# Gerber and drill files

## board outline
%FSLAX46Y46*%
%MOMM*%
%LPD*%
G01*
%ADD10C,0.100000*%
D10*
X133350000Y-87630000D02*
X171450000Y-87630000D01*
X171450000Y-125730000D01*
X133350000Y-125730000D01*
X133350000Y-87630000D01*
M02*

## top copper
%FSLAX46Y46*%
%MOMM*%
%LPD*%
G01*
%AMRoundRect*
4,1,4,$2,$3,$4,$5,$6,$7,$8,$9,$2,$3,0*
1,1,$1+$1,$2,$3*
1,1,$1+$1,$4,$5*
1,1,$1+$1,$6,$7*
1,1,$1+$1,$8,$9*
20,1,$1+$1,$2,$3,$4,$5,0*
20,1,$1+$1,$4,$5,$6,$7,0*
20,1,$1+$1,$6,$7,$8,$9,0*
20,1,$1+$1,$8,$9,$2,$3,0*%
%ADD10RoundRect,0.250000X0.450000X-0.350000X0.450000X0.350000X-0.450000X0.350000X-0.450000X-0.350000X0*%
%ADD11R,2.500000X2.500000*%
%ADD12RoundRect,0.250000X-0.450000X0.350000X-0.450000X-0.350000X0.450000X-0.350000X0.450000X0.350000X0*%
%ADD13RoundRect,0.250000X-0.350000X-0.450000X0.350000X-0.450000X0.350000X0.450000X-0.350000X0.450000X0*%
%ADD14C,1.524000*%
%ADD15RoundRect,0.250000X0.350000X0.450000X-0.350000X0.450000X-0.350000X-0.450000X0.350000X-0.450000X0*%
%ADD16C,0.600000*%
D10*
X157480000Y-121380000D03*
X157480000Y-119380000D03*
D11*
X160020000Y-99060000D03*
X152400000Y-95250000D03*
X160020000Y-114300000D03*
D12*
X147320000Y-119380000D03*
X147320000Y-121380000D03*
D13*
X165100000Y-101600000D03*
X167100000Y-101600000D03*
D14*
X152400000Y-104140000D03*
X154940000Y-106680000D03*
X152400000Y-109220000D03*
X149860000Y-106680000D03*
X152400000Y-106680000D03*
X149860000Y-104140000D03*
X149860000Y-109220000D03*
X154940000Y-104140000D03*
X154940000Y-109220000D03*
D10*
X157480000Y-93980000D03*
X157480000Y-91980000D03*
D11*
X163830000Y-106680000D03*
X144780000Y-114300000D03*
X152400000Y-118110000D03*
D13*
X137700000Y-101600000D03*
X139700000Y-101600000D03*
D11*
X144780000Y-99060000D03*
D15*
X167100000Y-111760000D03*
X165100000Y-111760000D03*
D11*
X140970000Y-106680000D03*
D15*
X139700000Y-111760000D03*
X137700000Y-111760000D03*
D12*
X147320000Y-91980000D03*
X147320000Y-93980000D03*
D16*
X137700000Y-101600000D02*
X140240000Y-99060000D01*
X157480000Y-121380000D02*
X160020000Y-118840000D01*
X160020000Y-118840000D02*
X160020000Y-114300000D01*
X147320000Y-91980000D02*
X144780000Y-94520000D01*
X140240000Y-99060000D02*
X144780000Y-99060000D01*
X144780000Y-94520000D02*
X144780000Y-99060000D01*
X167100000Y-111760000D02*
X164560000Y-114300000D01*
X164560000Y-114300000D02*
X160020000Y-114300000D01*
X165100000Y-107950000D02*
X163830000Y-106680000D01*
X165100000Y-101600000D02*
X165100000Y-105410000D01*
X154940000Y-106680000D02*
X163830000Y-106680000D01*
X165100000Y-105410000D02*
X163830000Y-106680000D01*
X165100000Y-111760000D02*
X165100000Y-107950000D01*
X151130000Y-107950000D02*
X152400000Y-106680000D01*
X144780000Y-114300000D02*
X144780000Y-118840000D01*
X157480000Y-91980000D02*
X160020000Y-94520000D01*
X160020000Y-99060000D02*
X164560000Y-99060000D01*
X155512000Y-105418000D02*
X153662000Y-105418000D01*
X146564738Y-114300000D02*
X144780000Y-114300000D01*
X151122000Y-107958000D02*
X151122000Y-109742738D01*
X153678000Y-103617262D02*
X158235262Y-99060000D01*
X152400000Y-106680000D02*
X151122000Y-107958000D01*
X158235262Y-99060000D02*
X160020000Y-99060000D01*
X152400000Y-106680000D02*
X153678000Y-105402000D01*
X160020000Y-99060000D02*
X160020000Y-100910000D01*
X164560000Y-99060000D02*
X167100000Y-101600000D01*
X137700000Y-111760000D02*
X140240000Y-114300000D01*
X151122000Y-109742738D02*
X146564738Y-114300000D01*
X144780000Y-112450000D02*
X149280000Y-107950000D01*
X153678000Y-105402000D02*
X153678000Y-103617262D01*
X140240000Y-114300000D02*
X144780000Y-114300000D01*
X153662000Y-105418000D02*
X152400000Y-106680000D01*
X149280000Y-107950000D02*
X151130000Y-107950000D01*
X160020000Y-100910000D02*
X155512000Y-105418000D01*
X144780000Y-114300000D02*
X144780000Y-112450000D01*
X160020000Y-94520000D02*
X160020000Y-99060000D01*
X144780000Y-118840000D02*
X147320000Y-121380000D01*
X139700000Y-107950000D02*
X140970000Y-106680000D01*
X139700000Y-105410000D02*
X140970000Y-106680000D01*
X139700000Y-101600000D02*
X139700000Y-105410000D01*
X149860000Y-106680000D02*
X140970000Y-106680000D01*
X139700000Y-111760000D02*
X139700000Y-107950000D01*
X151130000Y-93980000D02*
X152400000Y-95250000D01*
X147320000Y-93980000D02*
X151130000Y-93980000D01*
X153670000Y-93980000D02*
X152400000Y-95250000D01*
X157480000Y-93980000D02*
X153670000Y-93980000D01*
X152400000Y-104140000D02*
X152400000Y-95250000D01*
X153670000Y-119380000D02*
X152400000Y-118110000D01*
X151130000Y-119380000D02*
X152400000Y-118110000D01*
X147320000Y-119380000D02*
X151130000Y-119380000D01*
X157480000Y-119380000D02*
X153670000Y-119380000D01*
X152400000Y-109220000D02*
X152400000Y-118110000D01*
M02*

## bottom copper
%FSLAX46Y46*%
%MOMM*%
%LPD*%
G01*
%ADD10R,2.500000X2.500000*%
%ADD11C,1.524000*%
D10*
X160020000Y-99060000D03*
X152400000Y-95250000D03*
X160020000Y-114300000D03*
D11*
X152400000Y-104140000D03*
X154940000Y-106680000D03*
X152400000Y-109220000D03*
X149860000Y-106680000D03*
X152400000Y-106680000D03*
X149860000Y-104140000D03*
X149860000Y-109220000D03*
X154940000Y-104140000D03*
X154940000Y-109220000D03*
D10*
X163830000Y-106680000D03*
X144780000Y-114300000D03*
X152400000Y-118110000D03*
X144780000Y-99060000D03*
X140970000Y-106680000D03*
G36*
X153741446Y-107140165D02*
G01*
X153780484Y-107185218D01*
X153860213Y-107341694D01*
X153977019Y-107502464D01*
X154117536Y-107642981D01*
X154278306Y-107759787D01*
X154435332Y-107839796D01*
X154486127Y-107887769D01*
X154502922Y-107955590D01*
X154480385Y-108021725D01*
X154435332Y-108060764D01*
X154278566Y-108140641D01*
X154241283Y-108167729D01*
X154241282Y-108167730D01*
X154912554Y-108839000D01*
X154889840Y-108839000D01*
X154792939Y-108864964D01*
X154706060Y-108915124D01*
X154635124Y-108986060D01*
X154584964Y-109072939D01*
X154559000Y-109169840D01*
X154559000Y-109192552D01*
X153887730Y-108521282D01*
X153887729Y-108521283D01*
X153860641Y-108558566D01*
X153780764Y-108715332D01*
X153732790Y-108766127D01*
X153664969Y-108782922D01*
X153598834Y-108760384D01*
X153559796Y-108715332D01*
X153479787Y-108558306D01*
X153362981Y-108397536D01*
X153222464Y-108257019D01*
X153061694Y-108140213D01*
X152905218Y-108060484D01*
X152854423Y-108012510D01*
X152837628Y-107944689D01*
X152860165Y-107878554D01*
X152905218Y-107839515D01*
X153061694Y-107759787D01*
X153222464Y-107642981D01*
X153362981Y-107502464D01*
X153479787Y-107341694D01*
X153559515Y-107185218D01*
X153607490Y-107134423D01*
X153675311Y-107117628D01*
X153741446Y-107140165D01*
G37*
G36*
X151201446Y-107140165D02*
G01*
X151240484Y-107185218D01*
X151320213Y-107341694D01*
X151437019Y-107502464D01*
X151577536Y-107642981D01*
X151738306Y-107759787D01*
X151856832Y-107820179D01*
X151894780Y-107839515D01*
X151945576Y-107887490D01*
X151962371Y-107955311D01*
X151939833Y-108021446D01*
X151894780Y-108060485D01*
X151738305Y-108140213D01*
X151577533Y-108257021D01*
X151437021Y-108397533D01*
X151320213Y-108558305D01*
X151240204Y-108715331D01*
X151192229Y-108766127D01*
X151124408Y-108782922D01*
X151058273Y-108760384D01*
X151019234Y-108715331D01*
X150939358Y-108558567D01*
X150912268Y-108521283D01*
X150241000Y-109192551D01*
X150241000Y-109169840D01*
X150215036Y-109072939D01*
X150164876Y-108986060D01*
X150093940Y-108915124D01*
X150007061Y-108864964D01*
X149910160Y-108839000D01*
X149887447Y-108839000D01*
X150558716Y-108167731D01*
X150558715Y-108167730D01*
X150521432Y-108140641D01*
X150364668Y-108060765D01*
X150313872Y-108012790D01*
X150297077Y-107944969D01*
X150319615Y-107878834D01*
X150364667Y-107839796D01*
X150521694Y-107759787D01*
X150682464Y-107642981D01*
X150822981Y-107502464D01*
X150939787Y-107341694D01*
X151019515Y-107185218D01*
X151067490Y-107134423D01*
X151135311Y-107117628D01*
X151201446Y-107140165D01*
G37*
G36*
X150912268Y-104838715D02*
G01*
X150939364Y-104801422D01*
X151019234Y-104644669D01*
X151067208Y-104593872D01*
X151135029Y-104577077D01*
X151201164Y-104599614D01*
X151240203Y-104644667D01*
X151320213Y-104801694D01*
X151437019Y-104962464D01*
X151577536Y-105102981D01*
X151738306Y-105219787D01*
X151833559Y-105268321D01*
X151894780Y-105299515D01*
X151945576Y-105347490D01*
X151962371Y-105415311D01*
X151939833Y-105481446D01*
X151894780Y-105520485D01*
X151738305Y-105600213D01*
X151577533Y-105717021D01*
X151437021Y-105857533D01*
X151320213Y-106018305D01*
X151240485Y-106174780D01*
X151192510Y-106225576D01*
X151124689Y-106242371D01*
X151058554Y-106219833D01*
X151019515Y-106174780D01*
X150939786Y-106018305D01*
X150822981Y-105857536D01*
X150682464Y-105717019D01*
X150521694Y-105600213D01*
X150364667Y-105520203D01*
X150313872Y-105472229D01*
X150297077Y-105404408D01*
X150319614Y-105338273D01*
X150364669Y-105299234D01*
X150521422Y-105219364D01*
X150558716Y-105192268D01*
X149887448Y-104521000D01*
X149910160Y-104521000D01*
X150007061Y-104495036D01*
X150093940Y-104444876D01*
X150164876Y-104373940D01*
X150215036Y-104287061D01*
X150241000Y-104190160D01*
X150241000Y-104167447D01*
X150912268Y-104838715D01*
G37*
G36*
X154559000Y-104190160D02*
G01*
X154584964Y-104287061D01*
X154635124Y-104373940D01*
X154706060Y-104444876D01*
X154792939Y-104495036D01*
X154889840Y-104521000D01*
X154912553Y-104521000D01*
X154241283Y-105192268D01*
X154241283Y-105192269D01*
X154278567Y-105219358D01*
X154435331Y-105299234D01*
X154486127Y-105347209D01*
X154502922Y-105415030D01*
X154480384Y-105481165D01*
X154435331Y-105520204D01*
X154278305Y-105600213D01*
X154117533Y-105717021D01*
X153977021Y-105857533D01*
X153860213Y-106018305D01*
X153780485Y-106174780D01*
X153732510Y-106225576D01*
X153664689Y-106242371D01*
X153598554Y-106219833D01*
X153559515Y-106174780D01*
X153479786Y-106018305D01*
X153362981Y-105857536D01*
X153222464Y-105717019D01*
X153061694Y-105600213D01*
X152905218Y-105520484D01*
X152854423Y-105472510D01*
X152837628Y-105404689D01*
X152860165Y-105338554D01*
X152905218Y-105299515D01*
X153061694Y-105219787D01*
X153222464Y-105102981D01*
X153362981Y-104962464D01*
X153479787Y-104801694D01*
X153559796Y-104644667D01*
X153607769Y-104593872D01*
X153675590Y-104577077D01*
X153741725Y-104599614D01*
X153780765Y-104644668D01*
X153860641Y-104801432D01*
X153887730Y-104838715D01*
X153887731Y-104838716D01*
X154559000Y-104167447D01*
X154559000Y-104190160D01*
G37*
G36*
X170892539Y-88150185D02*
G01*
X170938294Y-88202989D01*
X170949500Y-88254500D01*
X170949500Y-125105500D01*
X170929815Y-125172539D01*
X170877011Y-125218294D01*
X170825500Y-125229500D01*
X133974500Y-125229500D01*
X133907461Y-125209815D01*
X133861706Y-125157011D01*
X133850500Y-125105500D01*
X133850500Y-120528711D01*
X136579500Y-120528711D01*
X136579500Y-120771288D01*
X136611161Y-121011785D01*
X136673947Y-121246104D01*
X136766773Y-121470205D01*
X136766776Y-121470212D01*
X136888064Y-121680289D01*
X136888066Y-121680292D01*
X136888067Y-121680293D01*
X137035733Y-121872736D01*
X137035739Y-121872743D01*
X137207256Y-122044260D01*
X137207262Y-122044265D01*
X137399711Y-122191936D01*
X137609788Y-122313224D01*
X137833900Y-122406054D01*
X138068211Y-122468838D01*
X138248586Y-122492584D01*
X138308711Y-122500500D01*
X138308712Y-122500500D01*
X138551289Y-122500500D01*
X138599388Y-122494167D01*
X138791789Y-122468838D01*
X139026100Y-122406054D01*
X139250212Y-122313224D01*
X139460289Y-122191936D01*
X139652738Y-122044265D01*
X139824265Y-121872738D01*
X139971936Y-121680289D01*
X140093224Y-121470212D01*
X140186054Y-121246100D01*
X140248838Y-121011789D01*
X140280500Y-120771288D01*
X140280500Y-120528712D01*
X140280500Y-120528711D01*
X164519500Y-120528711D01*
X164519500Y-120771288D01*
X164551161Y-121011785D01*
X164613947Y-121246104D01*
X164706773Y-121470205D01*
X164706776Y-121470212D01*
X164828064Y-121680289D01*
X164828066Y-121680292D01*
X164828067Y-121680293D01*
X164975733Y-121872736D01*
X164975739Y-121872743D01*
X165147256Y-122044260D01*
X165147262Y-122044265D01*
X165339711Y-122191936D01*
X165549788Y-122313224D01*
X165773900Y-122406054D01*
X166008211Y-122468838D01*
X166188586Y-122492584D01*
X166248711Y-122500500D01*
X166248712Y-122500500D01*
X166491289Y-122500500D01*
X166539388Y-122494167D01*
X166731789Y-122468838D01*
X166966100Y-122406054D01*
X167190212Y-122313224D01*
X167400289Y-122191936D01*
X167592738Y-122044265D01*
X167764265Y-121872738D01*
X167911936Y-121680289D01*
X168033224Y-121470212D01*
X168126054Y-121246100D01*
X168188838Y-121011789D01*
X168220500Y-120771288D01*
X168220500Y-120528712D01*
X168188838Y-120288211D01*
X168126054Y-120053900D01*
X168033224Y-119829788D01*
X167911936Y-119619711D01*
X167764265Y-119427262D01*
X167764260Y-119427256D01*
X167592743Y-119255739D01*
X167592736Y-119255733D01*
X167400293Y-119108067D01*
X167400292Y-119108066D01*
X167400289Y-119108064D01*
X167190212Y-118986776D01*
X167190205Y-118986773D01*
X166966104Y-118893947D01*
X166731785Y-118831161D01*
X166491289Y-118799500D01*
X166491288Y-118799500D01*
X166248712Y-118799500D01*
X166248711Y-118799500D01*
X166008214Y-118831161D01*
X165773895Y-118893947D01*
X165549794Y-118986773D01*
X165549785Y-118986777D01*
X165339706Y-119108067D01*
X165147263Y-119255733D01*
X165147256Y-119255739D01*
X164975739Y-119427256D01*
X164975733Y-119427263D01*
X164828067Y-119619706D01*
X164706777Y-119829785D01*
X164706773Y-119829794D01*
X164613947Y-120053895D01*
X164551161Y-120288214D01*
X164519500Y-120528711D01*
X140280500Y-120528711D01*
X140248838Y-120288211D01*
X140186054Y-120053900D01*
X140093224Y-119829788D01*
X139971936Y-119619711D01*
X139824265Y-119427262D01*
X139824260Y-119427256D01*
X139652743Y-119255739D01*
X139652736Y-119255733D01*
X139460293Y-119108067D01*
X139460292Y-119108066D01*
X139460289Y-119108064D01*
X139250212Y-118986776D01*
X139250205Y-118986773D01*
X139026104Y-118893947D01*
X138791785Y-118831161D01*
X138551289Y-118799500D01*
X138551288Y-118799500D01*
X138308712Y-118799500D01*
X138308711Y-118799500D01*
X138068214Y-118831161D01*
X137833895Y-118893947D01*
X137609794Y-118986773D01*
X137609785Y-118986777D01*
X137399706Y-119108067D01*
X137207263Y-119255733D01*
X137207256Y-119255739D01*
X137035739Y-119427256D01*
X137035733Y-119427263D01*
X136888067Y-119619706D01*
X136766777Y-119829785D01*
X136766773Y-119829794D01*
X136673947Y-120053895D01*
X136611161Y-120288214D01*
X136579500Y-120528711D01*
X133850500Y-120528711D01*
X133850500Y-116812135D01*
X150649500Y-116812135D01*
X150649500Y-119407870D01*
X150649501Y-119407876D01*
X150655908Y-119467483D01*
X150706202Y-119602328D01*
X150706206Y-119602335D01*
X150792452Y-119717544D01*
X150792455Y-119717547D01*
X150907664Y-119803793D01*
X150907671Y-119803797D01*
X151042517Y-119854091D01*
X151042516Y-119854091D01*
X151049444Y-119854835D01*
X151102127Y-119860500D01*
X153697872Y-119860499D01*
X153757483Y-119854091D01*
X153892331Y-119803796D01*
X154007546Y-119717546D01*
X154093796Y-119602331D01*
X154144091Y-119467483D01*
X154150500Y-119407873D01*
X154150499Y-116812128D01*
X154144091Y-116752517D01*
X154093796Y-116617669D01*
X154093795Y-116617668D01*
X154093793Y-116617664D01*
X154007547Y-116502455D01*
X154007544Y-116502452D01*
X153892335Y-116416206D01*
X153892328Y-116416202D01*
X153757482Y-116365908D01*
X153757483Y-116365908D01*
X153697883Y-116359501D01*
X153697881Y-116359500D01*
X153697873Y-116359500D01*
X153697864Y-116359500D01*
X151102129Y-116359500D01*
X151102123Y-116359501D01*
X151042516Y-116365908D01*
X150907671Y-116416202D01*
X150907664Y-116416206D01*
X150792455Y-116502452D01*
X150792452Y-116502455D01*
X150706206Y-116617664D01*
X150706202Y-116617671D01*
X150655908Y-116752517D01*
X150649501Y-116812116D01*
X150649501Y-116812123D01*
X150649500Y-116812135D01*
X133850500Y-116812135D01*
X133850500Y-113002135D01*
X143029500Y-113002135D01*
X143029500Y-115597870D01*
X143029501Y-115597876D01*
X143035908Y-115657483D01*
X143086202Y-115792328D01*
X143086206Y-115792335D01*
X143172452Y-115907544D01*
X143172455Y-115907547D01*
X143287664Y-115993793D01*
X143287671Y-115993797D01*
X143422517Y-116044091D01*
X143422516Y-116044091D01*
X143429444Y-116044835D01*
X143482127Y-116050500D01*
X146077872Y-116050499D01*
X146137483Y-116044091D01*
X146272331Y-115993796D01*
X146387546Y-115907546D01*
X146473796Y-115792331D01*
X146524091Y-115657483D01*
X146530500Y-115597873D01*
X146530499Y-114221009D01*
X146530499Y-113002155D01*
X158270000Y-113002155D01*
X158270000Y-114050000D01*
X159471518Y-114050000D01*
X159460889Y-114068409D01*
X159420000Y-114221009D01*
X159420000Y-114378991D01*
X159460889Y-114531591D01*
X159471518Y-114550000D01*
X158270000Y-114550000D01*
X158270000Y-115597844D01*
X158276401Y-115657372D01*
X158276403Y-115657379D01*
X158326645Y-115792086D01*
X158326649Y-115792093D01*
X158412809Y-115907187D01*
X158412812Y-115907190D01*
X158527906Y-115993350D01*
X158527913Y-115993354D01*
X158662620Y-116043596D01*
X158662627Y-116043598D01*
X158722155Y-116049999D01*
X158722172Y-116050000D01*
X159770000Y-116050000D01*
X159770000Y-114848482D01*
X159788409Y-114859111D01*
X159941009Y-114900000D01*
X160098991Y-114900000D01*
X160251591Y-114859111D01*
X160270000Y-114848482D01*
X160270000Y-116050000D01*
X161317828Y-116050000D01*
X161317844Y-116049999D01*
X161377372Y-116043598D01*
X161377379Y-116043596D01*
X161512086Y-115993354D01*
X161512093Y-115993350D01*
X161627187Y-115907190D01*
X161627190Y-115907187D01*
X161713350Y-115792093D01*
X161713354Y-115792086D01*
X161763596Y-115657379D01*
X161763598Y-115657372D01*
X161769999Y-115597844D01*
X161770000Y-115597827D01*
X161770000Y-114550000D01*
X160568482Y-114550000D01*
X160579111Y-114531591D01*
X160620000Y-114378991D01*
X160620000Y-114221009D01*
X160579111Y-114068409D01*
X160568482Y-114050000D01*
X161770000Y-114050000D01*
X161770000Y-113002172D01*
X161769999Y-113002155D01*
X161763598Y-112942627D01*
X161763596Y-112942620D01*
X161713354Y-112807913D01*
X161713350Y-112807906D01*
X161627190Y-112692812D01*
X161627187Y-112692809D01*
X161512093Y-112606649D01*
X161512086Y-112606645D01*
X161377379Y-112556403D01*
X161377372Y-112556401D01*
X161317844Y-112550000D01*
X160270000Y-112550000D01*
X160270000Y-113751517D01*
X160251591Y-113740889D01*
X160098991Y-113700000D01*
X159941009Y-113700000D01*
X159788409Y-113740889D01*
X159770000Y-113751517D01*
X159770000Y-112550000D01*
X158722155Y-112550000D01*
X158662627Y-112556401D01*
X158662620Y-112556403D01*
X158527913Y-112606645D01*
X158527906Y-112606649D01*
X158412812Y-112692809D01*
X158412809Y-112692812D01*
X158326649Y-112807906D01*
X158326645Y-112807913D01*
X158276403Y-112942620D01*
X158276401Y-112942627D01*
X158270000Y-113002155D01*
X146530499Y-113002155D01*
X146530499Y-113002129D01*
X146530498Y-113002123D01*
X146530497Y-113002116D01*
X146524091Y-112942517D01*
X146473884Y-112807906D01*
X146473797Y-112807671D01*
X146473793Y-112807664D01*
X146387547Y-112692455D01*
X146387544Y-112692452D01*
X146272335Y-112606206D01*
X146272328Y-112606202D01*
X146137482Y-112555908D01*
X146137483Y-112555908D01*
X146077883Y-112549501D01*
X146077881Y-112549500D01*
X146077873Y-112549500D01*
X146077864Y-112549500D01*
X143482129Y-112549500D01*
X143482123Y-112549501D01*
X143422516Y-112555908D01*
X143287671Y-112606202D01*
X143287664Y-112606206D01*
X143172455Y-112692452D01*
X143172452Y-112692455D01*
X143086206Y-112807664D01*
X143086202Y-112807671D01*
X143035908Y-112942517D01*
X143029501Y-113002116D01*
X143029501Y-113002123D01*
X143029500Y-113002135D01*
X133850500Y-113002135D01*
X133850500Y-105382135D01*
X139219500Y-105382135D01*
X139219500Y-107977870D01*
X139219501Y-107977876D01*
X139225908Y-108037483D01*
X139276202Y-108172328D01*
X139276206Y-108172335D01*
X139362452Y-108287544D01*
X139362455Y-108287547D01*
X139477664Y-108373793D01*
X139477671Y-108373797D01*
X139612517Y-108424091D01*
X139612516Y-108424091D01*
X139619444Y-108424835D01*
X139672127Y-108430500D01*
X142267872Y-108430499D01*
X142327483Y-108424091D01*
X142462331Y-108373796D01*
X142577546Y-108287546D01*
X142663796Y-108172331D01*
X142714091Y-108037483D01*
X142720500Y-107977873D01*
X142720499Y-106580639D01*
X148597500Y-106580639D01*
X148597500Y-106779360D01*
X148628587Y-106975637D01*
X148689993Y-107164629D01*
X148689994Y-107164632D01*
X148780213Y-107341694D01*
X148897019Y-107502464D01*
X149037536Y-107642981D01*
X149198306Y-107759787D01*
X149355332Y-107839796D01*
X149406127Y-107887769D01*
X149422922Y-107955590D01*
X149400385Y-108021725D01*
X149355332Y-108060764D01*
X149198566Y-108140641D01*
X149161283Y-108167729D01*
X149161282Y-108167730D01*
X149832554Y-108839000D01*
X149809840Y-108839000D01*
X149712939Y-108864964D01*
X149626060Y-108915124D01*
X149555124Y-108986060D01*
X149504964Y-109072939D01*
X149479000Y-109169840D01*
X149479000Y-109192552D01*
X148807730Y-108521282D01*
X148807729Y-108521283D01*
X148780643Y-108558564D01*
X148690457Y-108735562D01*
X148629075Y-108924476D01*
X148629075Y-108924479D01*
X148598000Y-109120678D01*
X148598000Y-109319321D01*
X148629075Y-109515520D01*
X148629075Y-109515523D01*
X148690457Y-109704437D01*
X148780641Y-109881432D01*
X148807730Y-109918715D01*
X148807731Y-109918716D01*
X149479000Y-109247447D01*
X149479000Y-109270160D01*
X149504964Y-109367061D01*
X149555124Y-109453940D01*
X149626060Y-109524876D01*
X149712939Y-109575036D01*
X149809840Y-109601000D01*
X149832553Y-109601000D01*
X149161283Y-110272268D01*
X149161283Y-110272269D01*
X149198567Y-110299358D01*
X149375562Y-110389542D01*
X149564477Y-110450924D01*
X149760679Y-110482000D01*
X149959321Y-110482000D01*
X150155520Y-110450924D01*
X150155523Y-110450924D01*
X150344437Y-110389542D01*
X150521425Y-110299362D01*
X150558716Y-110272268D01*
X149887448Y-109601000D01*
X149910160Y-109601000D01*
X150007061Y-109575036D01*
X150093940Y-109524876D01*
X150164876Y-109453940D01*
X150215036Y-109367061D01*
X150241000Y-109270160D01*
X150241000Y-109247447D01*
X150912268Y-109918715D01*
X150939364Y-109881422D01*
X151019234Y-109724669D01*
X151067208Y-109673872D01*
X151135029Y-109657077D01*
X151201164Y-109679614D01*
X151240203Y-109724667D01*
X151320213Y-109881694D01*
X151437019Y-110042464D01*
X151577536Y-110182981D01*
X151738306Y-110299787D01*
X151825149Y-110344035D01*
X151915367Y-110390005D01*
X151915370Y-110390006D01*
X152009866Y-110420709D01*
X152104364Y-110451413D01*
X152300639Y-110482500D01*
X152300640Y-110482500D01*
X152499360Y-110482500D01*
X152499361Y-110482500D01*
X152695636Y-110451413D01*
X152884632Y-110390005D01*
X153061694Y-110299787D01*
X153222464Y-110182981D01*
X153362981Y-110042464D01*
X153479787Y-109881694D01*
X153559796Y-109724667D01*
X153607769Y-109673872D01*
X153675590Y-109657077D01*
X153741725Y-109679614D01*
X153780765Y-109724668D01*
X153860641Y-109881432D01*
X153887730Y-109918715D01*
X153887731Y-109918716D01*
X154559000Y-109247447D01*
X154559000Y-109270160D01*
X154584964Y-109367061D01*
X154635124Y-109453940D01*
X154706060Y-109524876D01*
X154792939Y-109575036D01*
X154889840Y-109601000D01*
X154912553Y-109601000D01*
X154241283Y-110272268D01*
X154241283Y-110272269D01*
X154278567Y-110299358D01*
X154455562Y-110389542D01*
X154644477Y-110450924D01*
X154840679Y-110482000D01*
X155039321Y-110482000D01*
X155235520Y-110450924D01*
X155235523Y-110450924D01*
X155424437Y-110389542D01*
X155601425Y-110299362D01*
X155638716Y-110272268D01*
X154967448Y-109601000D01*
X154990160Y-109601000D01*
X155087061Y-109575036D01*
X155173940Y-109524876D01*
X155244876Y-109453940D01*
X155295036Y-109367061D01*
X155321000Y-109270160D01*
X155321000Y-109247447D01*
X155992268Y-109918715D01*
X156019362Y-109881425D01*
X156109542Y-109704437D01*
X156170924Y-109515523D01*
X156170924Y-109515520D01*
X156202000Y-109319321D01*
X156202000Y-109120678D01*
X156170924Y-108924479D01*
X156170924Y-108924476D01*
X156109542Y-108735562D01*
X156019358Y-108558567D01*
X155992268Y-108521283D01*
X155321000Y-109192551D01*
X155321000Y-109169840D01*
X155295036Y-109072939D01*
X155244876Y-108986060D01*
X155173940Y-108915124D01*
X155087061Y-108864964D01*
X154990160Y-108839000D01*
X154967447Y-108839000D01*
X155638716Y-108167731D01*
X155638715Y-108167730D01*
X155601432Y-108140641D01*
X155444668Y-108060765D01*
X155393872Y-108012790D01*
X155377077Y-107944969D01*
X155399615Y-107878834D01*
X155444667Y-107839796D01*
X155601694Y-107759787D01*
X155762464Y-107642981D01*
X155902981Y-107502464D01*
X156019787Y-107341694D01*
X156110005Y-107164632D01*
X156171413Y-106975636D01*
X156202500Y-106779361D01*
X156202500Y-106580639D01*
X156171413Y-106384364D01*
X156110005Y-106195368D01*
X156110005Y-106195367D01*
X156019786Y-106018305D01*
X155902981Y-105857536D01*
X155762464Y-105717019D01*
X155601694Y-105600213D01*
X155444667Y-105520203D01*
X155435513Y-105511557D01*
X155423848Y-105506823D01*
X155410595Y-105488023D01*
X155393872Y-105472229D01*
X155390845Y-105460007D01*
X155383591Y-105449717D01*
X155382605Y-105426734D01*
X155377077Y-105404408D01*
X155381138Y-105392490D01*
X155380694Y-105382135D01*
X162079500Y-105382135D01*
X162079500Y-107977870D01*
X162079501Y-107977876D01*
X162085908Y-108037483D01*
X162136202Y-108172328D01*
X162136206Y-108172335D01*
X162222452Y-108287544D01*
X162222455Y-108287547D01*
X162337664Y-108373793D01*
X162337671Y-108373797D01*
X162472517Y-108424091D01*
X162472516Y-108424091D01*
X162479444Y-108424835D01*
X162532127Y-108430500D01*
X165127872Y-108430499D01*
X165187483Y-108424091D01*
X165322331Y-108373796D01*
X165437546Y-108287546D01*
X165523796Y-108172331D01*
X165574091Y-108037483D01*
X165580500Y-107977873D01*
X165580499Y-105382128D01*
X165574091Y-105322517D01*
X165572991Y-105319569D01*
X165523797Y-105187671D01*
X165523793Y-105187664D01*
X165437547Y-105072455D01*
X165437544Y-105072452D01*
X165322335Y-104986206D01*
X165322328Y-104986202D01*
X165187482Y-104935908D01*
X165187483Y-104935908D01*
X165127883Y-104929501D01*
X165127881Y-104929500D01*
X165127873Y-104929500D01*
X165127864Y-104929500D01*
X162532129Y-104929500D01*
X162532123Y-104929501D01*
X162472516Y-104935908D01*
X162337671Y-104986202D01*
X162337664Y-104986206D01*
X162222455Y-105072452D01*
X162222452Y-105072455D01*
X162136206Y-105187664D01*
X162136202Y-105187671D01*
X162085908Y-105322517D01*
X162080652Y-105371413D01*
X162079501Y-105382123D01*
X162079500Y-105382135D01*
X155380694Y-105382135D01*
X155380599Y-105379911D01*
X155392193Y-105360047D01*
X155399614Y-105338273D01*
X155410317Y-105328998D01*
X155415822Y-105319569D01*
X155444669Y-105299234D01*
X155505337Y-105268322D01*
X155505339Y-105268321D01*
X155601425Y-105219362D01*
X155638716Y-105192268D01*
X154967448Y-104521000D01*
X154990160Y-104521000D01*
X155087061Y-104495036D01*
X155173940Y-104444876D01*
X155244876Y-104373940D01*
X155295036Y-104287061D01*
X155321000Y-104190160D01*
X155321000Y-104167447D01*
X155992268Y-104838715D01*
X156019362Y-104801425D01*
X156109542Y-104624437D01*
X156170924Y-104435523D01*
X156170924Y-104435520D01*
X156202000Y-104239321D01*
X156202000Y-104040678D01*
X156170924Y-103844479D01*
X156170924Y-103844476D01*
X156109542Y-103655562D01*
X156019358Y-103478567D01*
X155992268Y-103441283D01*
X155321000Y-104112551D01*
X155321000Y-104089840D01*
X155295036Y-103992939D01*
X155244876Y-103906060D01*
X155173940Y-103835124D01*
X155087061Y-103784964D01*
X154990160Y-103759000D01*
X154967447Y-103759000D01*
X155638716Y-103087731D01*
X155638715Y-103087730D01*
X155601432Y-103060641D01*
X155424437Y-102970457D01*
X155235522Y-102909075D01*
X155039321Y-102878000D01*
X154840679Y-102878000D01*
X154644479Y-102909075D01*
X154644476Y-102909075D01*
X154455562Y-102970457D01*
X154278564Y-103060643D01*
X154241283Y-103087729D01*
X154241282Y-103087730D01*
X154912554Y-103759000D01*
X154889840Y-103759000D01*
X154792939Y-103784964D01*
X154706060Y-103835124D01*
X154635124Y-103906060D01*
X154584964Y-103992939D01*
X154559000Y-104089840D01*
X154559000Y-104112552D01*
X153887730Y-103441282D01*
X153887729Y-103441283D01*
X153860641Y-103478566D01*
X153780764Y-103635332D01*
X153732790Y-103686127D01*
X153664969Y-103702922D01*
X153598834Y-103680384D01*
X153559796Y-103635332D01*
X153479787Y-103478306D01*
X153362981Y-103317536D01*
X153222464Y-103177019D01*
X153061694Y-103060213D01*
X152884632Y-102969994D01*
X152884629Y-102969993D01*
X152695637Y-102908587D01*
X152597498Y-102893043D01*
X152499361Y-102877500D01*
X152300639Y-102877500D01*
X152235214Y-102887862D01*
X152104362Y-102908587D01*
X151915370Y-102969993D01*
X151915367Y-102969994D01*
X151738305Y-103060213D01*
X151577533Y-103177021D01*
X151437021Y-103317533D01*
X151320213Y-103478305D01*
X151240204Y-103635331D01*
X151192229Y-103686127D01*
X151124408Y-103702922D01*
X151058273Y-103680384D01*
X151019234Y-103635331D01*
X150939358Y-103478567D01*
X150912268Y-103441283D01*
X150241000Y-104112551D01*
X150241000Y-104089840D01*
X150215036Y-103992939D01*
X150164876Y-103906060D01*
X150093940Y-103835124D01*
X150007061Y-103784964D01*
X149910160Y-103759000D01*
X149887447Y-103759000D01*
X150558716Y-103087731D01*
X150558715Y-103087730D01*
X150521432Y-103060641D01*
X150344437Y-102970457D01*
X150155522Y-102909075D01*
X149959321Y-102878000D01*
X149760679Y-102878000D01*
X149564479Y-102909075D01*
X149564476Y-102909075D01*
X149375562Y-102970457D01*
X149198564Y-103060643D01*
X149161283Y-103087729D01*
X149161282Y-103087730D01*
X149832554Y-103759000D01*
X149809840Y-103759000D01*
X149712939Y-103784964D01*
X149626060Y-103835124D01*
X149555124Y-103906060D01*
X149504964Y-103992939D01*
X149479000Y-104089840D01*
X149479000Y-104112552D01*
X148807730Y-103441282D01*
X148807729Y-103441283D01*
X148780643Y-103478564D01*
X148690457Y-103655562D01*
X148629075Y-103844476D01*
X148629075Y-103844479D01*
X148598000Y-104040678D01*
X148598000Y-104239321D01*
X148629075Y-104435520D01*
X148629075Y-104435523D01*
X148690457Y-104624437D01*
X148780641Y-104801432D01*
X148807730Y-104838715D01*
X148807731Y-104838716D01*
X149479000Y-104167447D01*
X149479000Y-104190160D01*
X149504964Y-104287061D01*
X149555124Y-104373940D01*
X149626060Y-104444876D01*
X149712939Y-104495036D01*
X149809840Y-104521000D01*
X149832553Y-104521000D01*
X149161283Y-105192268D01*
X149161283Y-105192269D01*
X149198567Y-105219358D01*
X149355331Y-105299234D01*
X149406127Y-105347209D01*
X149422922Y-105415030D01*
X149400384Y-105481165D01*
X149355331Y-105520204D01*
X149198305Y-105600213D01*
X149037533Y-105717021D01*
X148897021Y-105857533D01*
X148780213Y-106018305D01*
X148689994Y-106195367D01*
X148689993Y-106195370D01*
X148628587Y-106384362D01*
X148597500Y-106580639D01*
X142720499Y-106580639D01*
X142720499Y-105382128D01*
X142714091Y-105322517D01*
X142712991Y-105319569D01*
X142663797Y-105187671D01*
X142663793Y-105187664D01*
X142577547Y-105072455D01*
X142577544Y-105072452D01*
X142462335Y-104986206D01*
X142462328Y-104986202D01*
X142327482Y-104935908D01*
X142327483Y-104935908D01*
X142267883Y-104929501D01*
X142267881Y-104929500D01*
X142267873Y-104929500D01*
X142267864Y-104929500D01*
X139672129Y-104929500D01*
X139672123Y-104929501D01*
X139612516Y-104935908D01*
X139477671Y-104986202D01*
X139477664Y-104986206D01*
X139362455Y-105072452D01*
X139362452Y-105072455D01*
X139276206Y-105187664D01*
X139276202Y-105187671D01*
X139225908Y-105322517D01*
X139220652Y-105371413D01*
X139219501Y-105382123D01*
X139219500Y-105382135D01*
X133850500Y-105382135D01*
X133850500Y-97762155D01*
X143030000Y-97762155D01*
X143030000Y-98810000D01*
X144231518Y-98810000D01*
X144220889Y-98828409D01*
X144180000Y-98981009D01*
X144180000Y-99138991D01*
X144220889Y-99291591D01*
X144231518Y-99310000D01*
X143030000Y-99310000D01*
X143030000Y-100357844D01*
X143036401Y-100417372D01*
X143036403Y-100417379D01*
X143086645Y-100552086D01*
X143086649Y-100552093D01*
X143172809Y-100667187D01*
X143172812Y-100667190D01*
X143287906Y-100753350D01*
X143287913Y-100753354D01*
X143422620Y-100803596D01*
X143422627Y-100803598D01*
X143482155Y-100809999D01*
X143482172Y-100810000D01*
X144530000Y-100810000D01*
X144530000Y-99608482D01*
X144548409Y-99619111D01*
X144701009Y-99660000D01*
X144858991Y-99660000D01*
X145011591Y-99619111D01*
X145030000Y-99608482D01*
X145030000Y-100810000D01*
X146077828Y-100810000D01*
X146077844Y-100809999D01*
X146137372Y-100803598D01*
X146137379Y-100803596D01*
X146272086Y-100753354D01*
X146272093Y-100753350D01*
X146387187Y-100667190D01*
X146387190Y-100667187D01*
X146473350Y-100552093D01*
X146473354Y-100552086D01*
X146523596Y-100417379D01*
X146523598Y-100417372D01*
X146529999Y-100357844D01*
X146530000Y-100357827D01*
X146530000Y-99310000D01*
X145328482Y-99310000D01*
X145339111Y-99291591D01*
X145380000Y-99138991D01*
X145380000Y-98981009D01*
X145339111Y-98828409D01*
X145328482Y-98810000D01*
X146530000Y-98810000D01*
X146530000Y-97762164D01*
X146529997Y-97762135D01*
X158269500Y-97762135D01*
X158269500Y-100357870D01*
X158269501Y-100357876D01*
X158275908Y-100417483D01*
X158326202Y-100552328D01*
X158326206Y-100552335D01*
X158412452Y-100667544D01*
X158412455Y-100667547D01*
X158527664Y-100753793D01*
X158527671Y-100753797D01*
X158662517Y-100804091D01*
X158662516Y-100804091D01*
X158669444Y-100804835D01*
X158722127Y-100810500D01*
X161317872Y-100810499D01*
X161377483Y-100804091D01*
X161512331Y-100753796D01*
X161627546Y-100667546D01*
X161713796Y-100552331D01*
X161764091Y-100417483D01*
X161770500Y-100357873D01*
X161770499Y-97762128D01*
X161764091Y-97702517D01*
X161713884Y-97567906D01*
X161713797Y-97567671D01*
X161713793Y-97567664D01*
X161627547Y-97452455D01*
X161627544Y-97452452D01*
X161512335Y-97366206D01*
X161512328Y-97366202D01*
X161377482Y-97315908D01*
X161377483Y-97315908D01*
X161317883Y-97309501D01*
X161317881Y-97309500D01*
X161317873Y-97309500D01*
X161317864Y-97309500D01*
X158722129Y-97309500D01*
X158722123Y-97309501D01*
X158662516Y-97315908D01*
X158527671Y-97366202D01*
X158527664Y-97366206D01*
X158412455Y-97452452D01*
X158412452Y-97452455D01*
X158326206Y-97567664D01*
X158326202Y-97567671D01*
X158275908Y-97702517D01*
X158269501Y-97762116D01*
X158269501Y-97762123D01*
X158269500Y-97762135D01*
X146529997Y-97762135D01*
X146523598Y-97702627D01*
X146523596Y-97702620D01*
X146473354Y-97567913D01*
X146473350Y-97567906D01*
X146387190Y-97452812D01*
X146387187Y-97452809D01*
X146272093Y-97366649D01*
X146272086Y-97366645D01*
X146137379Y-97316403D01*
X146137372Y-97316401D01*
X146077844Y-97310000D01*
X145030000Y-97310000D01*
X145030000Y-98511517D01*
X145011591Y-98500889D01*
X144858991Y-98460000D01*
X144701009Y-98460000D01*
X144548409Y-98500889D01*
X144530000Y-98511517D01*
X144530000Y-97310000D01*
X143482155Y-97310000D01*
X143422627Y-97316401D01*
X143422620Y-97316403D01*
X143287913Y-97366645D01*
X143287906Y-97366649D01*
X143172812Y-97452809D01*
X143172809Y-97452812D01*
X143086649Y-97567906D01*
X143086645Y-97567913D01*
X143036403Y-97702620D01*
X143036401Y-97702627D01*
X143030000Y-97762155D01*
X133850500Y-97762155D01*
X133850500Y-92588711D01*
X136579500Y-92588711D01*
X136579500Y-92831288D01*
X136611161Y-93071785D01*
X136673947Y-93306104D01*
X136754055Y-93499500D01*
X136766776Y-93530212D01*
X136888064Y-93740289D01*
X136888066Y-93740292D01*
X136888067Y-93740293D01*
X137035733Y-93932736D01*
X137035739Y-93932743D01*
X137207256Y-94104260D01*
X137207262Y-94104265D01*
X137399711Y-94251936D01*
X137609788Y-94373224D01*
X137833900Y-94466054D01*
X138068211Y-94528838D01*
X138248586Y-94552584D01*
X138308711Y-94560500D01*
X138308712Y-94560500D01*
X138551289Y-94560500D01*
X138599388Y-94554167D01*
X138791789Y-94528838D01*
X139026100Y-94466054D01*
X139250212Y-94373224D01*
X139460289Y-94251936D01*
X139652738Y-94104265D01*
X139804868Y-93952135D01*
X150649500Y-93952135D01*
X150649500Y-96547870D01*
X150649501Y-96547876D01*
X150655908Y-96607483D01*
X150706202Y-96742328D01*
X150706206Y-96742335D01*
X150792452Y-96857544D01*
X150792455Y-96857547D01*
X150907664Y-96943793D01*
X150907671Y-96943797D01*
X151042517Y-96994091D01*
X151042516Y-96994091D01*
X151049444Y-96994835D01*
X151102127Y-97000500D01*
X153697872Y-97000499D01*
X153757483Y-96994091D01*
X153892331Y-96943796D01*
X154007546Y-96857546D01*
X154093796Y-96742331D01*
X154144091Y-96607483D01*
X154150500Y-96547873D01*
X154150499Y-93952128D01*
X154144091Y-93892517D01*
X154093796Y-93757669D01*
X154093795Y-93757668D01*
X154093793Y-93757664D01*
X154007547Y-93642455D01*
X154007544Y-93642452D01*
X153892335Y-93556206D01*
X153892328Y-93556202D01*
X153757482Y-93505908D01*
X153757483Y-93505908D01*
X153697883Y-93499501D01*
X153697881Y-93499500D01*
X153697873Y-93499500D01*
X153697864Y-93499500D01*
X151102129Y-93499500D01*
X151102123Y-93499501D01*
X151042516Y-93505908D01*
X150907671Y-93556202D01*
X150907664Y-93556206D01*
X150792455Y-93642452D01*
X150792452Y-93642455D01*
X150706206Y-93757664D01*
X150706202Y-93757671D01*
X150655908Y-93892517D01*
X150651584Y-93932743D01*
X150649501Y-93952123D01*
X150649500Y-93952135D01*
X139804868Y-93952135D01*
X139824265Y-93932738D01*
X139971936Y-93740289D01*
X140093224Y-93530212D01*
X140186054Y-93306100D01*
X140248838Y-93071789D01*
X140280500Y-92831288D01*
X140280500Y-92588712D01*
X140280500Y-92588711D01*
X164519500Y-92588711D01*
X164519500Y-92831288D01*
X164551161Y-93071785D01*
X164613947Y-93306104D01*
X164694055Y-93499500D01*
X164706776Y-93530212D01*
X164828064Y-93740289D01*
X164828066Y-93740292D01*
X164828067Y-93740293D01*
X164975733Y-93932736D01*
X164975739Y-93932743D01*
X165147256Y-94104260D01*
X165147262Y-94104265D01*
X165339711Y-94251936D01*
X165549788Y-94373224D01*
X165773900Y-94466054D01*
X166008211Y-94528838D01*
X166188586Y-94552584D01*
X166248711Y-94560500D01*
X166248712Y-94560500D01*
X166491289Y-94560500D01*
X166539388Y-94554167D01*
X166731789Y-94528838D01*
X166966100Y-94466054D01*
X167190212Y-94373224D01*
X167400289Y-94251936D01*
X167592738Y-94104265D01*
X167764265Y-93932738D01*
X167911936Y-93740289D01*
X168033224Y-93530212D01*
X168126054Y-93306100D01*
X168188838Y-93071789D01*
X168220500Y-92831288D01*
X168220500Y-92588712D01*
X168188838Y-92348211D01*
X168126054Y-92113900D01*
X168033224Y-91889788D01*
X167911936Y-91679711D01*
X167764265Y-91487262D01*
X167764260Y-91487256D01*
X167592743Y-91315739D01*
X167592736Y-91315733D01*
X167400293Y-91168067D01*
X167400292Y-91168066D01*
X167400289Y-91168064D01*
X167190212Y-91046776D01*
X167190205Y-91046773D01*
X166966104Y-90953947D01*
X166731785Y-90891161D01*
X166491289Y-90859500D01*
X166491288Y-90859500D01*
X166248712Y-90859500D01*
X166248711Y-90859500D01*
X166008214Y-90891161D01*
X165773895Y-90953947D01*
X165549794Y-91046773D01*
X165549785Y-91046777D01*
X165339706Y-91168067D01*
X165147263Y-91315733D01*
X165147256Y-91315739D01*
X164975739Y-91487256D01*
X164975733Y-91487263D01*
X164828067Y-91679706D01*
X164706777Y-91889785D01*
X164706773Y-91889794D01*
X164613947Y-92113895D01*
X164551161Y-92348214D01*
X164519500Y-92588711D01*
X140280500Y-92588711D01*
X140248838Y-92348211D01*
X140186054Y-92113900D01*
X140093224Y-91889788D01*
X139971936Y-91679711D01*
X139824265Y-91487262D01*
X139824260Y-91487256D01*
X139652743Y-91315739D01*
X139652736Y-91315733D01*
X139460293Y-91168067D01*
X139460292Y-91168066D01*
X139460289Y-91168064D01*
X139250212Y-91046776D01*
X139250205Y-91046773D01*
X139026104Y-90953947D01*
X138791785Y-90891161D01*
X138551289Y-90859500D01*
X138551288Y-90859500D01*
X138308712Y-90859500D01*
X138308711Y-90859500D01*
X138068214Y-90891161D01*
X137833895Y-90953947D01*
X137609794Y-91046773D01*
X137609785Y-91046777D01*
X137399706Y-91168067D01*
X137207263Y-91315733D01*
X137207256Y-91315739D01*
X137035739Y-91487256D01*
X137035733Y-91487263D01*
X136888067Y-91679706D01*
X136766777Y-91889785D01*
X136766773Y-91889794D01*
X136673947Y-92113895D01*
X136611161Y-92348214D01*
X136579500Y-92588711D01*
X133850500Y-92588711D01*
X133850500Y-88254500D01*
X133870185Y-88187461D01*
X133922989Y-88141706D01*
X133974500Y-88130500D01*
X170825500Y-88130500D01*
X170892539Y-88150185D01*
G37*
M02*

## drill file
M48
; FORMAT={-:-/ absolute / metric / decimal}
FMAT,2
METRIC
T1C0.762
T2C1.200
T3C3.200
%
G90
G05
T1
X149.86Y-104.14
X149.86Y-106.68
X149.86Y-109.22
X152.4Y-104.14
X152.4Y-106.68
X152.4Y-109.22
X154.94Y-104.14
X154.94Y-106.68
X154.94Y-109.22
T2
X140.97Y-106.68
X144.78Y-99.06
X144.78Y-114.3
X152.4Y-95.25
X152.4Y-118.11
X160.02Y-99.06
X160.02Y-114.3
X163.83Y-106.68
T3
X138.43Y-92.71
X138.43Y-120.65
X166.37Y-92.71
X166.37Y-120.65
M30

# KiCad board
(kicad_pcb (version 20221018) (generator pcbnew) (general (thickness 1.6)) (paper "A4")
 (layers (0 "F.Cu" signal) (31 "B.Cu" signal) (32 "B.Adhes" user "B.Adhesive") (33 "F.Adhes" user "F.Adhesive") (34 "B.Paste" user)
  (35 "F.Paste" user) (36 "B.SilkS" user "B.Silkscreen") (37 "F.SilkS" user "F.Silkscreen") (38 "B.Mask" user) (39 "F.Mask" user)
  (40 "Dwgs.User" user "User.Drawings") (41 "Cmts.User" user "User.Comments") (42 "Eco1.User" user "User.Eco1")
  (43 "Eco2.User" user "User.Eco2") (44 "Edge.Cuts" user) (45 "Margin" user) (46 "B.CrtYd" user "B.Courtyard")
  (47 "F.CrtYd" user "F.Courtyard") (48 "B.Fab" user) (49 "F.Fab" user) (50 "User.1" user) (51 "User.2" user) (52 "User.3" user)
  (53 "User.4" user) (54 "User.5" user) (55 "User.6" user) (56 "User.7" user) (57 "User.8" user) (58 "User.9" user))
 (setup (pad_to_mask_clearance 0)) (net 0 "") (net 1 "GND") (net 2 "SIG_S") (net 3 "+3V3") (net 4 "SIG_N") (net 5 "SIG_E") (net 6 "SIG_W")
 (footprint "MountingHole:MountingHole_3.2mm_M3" (layer "F.Cu") (at 138.43 92.71)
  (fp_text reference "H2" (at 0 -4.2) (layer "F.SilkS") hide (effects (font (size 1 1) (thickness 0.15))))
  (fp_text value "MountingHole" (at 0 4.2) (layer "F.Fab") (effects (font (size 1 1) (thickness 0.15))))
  (pad "" np_thru_hole circle (at 0 0) (size 3.2 3.2) (drill 3.2) (layers "*.Cu" "*.Mask")))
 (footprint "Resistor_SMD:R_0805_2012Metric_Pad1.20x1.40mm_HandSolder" (layer "F.Cu") (at 157.48 120.38 90)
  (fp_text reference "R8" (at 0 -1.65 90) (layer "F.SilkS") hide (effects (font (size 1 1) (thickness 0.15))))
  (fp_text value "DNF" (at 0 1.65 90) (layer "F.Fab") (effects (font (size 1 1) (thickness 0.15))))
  (pad "1" smd roundrect (at -1 0 90) (size 1.2 1.4) (layers "F.Cu" "F.Paste" "F.Mask") (roundrect_rratio 0.2083333333) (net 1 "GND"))
  (pad "2" smd roundrect (at 1 0 90) (size 1.2 1.4) (layers "F.Cu" "F.Paste" "F.Mask") (roundrect_rratio 0.2083333333) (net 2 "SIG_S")))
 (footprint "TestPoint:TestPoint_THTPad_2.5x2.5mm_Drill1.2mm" (layer "F.Cu") (at 160.02 99.06)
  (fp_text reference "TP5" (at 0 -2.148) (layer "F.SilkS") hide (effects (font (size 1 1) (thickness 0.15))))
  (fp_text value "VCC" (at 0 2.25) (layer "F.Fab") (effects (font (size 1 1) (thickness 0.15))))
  (pad "1" thru_hole rect (at 0 0) (size 2.5 2.5) (drill 1.2) (layers "*.Cu" "*.Mask") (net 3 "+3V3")))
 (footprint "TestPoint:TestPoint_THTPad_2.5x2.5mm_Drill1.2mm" (layer "F.Cu") (at 152.4 95.25)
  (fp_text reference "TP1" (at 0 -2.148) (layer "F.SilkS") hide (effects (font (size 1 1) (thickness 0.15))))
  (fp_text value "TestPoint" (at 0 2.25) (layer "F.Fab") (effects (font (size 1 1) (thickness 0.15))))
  (pad "1" thru_hole rect (at 0 0) (size 2.5 2.5) (drill 1.2) (layers "*.Cu" "*.Mask") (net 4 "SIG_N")))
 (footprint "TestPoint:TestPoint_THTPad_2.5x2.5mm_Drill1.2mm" (layer "F.Cu") (at 160.02 114.3)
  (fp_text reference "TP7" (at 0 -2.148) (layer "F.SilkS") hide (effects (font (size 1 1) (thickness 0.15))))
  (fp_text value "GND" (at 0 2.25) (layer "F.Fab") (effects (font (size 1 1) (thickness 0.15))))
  (pad "1" thru_hole rect (at 0 0) (size 2.5 2.5) (drill 1.2) (layers "*.Cu" "*.Mask") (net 1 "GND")))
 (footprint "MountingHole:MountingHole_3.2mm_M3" (layer "F.Cu") (at 166.37 92.71)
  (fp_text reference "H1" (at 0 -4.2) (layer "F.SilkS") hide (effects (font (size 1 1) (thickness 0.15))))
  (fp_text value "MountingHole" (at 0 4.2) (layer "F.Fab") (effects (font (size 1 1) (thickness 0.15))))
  (pad "" np_thru_hole circle (at 0 0) (size 3.2 3.2) (drill 3.2) (layers "*.Cu" "*.Mask")))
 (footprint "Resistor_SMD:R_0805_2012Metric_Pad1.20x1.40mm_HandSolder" (layer "F.Cu") (at 147.32 120.38 -90)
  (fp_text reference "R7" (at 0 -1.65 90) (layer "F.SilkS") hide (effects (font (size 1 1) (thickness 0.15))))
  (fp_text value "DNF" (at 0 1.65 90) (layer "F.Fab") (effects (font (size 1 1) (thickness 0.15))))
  (pad "1" smd roundrect (at -1 0 270) (size 1.2 1.4) (layers "F.Cu" "F.Paste" "F.Mask") (roundrect_rratio 0.2083333333) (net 2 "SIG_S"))
  (pad "2" smd roundrect (at 1 0 270) (size 1.2 1.4) (layers "F.Cu" "F.Paste" "F.Mask") (roundrect_rratio 0.2083333333) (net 3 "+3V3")))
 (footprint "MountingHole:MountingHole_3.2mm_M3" (layer "F.Cu") (at 138.43 120.65)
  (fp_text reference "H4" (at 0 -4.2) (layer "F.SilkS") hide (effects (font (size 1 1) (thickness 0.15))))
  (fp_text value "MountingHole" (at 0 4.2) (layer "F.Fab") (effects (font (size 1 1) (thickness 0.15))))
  (pad "" np_thru_hole circle (at 0 0) (size 3.2 3.2) (drill 3.2) (layers "*.Cu" "*.Mask")))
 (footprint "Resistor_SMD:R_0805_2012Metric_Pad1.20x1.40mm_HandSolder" (layer "F.Cu") (at 166.1 101.6)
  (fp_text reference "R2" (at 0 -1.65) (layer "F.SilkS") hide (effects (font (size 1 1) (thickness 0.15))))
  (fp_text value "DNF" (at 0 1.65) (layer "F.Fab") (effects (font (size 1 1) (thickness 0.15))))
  (pad "1" smd roundrect (at -1 0) (size 1.2 1.4) (layers "F.Cu" "F.Paste" "F.Mask") (roundrect_rratio 0.2083333333) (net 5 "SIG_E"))
  (pad "2" smd roundrect (at 1 0) (size 1.2 1.4) (layers "F.Cu" "F.Paste" "F.Mask") (roundrect_rratio 0.2083333333) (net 3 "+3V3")))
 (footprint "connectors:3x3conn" (layer "F.Cu") (at 152.4 106.68)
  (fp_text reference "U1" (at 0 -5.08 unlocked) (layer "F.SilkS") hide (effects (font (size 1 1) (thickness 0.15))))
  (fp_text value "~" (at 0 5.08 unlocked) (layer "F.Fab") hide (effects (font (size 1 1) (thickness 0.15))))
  (pad "1" thru_hole circle (at 0 -2.54) (size 1.524 1.524) (drill 0.762) (layers "*.Cu" "*.Mask") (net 4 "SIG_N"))
  (pad "2" thru_hole circle (at 2.54 0) (size 1.524 1.524) (drill 0.762) (layers "*.Cu" "*.Mask") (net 5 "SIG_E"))
  (pad "3" thru_hole circle (at 0 2.54) (size 1.524 1.524) (drill 0.762) (layers "*.Cu" "*.Mask") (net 2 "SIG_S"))
  (pad "4" thru_hole circle (at -2.54 0) (size 1.524 1.524) (drill 0.762) (layers "*.Cu" "*.Mask") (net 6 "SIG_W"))
  (pad "5" thru_hole circle (at 0 0) (size 1.524 1.524) (drill 0.762) (layers "*.Cu" "*.Mask") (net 3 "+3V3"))
  (pad "6" thru_hole circle (at -2.54 -2.54) (size 1.524 1.524) (drill 0.762) (layers "*.Cu" "*.Mask") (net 1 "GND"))
  (pad "6" thru_hole circle (at -2.54 2.54) (size 1.524 1.524) (drill 0.762) (layers "*.Cu" "*.Mask") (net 1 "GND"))
  (pad "6" thru_hole circle (at 2.54 -2.54) (size 1.524 1.524) (drill 0.762) (layers "*.Cu" "*.Mask") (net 1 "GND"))
  (pad "6" thru_hole circle (at 2.54 2.54) (size 1.524 1.524) (drill 0.762) (layers "*.Cu" "*.Mask") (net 1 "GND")))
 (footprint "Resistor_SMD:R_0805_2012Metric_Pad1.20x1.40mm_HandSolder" (layer "F.Cu") (at 157.48 92.98 90)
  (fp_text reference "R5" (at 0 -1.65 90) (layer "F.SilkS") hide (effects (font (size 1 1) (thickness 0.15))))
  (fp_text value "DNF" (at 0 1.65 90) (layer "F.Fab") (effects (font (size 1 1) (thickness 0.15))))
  (pad "1" smd roundrect (at -1 0 90) (size 1.2 1.4) (layers "F.Cu" "F.Paste" "F.Mask") (roundrect_rratio 0.2083333333) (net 4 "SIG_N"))
  (pad "2" smd roundrect (at 1 0 90) (size 1.2 1.4) (layers "F.Cu" "F.Paste" "F.Mask") (roundrect_rratio 0.2083333333) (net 3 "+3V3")))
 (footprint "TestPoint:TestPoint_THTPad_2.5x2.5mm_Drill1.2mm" (layer "F.Cu") (at 163.83 106.68)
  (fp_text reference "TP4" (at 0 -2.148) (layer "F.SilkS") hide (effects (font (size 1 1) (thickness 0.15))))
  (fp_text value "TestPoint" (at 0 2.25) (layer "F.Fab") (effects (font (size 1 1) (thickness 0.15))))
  (pad "1" thru_hole rect (at 0 0) (size 2.5 2.5) (drill 1.2) (layers "*.Cu" "*.Mask") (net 5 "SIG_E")))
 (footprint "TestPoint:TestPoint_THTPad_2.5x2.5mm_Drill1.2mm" (layer "F.Cu") (at 144.78 114.3)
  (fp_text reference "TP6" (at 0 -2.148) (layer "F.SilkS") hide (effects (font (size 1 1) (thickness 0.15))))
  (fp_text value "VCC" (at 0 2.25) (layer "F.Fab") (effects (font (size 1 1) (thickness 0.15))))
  (pad "1" thru_hole rect (at 0 0) (size 2.5 2.5) (drill 1.2) (layers "*.Cu" "*.Mask") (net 3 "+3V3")))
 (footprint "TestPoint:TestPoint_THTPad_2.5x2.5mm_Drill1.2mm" (layer "F.Cu") (at 152.4 118.11)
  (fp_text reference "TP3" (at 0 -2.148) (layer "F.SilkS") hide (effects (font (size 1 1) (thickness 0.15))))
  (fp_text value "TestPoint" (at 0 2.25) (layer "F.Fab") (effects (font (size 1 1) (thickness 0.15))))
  (pad "1" thru_hole rect (at 0 0) (size 2.5 2.5) (drill 1.2) (layers "*.Cu" "*.Mask") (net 2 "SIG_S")))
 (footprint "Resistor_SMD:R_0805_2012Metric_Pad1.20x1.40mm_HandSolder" (layer "F.Cu") (at 138.7 101.6)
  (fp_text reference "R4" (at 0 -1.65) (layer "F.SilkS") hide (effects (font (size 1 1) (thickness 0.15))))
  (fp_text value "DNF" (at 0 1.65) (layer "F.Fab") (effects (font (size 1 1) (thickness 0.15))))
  (pad "1" smd roundrect (at -1 0) (size 1.2 1.4) (layers "F.Cu" "F.Paste" "F.Mask") (roundrect_rratio 0.2083333333) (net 1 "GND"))
  (pad "2" smd roundrect (at 1 0) (size 1.2 1.4) (layers "F.Cu" "F.Paste" "F.Mask") (roundrect_rratio 0.2083333333) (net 6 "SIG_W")))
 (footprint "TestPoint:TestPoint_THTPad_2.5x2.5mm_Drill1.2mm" (layer "F.Cu") (at 144.78 99.06)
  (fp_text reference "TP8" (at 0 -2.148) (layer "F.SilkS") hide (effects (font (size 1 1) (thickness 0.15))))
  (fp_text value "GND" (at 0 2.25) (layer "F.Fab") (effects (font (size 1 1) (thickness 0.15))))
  (pad "1" thru_hole rect (at 0 0) (size 2.5 2.5) (drill 1.2) (layers "*.Cu" "*.Mask") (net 1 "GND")))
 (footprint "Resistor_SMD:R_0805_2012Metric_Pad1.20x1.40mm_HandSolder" (layer "F.Cu") (at 166.1 111.76 180)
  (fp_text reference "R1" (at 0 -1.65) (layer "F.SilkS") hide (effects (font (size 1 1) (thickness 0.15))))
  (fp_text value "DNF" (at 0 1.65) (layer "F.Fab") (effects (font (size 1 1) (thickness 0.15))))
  (pad "1" smd roundrect (at -1 0 180) (size 1.2 1.4) (layers "F.Cu" "F.Paste" "F.Mask") (roundrect_rratio 0.2083333333) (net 1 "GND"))
  (pad "2" smd roundrect (at 1 0 180) (size 1.2 1.4) (layers "F.Cu" "F.Paste" "F.Mask") (roundrect_rratio 0.2083333333) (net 5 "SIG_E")))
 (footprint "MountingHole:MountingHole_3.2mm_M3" (layer "F.Cu") (at 166.37 120.65)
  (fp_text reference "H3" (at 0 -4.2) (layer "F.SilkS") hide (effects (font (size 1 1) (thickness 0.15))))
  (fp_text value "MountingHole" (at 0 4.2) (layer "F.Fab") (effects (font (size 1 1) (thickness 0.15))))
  (pad "" np_thru_hole circle (at 0 0) (size 3.2 3.2) (drill 3.2) (layers "*.Cu" "*.Mask")))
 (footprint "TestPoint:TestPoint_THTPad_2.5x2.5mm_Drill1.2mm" (layer "F.Cu") (at 140.97 106.68)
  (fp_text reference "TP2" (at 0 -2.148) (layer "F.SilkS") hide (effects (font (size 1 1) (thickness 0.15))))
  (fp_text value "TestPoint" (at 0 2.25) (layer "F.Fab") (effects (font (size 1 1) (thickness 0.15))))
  (pad "1" thru_hole rect (at 0 0) (size 2.5 2.5) (drill 1.2) (layers "*.Cu" "*.Mask") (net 6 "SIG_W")))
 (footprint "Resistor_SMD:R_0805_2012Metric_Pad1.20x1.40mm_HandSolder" (layer "F.Cu") (at 138.7 111.76 180)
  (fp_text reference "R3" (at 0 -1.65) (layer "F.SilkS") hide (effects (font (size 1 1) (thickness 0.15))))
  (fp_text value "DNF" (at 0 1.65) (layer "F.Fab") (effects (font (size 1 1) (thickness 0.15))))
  (pad "1" smd roundrect (at -1 0 180) (size 1.2 1.4) (layers "F.Cu" "F.Paste" "F.Mask") (roundrect_rratio 0.2083333333) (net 6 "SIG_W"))
  (pad "2" smd roundrect (at 1 0 180) (size 1.2 1.4) (layers "F.Cu" "F.Paste" "F.Mask") (roundrect_rratio 0.2083333333) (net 3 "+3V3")))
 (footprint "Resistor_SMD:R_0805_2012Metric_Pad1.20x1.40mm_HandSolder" (layer "F.Cu") (at 147.32 92.98 -90)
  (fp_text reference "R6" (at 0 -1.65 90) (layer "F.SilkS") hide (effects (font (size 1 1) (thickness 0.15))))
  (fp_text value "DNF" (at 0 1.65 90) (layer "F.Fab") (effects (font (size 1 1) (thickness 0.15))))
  (pad "1" smd roundrect (at -1 0 270) (size 1.2 1.4) (layers "F.Cu" "F.Paste" "F.Mask") (roundrect_rratio 0.2083333333) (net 1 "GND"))
  (pad "2" smd roundrect (at 1 0 270) (size 1.2 1.4) (layers "F.Cu" "F.Paste" "F.Mask") (roundrect_rratio 0.2083333333) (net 4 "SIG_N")))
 (gr_rect (start 133.35 87.63) (end 171.45 125.73) (stroke (width 0.1) (type default)) (fill none) (layer "Edge.Cuts"))
 (segment (start 137.7 101.6) (end 140.24 99.06) (width 0.6) (layer "F.Cu") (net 1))
 (segment (start 157.48 121.38) (end 160.02 118.84) (width 0.6) (layer "F.Cu") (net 1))
 (segment (start 160.02 118.84) (end 160.02 114.3) (width 0.6) (layer "F.Cu") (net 1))
 (segment (start 147.32 91.98) (end 144.78 94.52) (width 0.6) (layer "F.Cu") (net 1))
 (segment (start 140.24 99.06) (end 144.78 99.06) (width 0.6) (layer "F.Cu") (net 1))
 (segment (start 144.78 94.52) (end 144.78 99.06) (width 0.6) (layer "F.Cu") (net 1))
 (segment (start 167.1 111.76) (end 164.56 114.3) (width 0.6) (layer "F.Cu") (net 1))
 (segment (start 164.56 114.3) (end 160.02 114.3) (width 0.6) (layer "F.Cu") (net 1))
 (segment (start 165.1 107.95) (end 163.83 106.68) (width 0.6) (layer "F.Cu") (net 5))
 (segment (start 165.1 101.6) (end 165.1 105.41) (width 0.6) (layer "F.Cu") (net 5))
 (segment (start 154.94 106.68) (end 163.83 106.68) (width 0.6) (layer "F.Cu") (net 5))
 (segment (start 165.1 105.41) (end 163.83 106.68) (width 0.6) (layer "F.Cu") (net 5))
 (segment (start 165.1 111.76) (end 165.1 107.95) (width 0.6) (layer "F.Cu") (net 5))
 (segment (start 151.13 107.95) (end 152.4 106.68) (width 0.6) (layer "F.Cu") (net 3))
 (segment (start 144.78 114.3) (end 144.78 118.84) (width 0.6) (layer "F.Cu") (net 3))
 (segment (start 157.48 91.98) (end 160.02 94.52) (width 0.6) (layer "F.Cu") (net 3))
 (segment (start 160.02 99.06) (end 164.56 99.06) (width 0.6) (layer "F.Cu") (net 3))
 (segment (start 155.512 105.418) (end 153.662 105.418) (width 0.6) (layer "F.Cu") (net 3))
 (segment (start 146.564738 114.3) (end 144.78 114.3) (width 0.6) (layer "F.Cu") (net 3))
 (segment (start 151.122 107.958) (end 151.122 109.742738) (width 0.6) (layer "F.Cu") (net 3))
 (segment (start 153.678 103.617262) (end 158.235262 99.06) (width 0.6) (layer "F.Cu") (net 3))
 (segment (start 152.4 106.68) (end 151.122 107.958) (width 0.6) (layer "F.Cu") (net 3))
 (segment (start 158.235262 99.06) (end 160.02 99.06) (width 0.6) (layer "F.Cu") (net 3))
 (segment (start 152.4 106.68) (end 153.678 105.402) (width 0.6) (layer "F.Cu") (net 3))
 (segment (start 160.02 99.06) (end 160.02 100.91) (width 0.6) (layer "F.Cu") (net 3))
 (segment (start 164.56 99.06) (end 167.1 101.6) (width 0.6) (layer "F.Cu") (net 3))
 (segment (start 137.7 111.76) (end 140.24 114.3) (width 0.6) (layer "F.Cu") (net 3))
 (segment (start 151.122 109.742738) (end 146.564738 114.3) (width 0.6) (layer "F.Cu") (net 3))
 (segment (start 144.78 112.45) (end 149.28 107.95) (width 0.6) (layer "F.Cu") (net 3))
 (segment (start 153.678 105.402) (end 153.678 103.617262) (width 0.6) (layer "F.Cu") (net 3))
 (segment (start 140.24 114.3) (end 144.78 114.3) (width 0.6) (layer "F.Cu") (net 3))
 (segment (start 153.662 105.418) (end 152.4 106.68) (width 0.6) (layer "F.Cu") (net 3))
 (segment (start 149.28 107.95) (end 151.13 107.95) (width 0.6) (layer "F.Cu") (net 3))
 (segment (start 160.02 100.91) (end 155.512 105.418) (width 0.6) (layer "F.Cu") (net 3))
 (segment (start 144.78 114.3) (end 144.78 112.45) (width 0.6) (layer "F.Cu") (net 3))
 (segment (start 160.02 94.52) (end 160.02 99.06) (width 0.6) (layer "F.Cu") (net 3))
 (segment (start 144.78 118.84) (end 147.32 121.38) (width 0.6) (layer "F.Cu") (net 3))
 (segment (start 139.7 107.95) (end 140.97 106.68) (width 0.6) (layer "F.Cu") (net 6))
 (segment (start 139.7 105.41) (end 140.97 106.68) (width 0.6) (layer "F.Cu") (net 6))
 (segment (start 139.7 101.6) (end 139.7 105.41) (width 0.6) (layer "F.Cu") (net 6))
 (segment (start 149.86 106.68) (end 140.97 106.68) (width 0.6) (layer "F.Cu") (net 6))
 (segment (start 139.7 111.76) (end 139.7 107.95) (width 0.6) (layer "F.Cu") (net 6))
 (segment (start 151.13 93.98) (end 152.4 95.25) (width 0.6) (layer "F.Cu") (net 4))
 (segment (start 147.32 93.98) (end 151.13 93.98) (width 0.6) (layer "F.Cu") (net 4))
 (segment (start 153.67 93.98) (end 152.4 95.25) (width 0.6) (layer "F.Cu") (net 4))
 (segment (start 157.48 93.98) (end 153.67 93.98) (width 0.6) (layer "F.Cu") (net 4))
 (segment (start 152.4 104.14) (end 152.4 95.25) (width 0.6) (layer "F.Cu") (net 4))
 (segment (start 153.67 119.38) (end 152.4 118.11) (width 0.6) (layer "F.Cu") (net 2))
 (segment (start 151.13 119.38) (end 152.4 118.11) (width 0.6) (layer "F.Cu") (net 2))
 (segment (start 147.32 119.38) (end 151.13 119.38) (width 0.6) (layer "F.Cu") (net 2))
 (segment (start 157.48 119.38) (end 153.67 119.38) (width 0.6) (layer "F.Cu") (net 2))
 (segment (start 152.4 109.22) (end 152.4 118.11) (width 0.6) (layer "F.Cu") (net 2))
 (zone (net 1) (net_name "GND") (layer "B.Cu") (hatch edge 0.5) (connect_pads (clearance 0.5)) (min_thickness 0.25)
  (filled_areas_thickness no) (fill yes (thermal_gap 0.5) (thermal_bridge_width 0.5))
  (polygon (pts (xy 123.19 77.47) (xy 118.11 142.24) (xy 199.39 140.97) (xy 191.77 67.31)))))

